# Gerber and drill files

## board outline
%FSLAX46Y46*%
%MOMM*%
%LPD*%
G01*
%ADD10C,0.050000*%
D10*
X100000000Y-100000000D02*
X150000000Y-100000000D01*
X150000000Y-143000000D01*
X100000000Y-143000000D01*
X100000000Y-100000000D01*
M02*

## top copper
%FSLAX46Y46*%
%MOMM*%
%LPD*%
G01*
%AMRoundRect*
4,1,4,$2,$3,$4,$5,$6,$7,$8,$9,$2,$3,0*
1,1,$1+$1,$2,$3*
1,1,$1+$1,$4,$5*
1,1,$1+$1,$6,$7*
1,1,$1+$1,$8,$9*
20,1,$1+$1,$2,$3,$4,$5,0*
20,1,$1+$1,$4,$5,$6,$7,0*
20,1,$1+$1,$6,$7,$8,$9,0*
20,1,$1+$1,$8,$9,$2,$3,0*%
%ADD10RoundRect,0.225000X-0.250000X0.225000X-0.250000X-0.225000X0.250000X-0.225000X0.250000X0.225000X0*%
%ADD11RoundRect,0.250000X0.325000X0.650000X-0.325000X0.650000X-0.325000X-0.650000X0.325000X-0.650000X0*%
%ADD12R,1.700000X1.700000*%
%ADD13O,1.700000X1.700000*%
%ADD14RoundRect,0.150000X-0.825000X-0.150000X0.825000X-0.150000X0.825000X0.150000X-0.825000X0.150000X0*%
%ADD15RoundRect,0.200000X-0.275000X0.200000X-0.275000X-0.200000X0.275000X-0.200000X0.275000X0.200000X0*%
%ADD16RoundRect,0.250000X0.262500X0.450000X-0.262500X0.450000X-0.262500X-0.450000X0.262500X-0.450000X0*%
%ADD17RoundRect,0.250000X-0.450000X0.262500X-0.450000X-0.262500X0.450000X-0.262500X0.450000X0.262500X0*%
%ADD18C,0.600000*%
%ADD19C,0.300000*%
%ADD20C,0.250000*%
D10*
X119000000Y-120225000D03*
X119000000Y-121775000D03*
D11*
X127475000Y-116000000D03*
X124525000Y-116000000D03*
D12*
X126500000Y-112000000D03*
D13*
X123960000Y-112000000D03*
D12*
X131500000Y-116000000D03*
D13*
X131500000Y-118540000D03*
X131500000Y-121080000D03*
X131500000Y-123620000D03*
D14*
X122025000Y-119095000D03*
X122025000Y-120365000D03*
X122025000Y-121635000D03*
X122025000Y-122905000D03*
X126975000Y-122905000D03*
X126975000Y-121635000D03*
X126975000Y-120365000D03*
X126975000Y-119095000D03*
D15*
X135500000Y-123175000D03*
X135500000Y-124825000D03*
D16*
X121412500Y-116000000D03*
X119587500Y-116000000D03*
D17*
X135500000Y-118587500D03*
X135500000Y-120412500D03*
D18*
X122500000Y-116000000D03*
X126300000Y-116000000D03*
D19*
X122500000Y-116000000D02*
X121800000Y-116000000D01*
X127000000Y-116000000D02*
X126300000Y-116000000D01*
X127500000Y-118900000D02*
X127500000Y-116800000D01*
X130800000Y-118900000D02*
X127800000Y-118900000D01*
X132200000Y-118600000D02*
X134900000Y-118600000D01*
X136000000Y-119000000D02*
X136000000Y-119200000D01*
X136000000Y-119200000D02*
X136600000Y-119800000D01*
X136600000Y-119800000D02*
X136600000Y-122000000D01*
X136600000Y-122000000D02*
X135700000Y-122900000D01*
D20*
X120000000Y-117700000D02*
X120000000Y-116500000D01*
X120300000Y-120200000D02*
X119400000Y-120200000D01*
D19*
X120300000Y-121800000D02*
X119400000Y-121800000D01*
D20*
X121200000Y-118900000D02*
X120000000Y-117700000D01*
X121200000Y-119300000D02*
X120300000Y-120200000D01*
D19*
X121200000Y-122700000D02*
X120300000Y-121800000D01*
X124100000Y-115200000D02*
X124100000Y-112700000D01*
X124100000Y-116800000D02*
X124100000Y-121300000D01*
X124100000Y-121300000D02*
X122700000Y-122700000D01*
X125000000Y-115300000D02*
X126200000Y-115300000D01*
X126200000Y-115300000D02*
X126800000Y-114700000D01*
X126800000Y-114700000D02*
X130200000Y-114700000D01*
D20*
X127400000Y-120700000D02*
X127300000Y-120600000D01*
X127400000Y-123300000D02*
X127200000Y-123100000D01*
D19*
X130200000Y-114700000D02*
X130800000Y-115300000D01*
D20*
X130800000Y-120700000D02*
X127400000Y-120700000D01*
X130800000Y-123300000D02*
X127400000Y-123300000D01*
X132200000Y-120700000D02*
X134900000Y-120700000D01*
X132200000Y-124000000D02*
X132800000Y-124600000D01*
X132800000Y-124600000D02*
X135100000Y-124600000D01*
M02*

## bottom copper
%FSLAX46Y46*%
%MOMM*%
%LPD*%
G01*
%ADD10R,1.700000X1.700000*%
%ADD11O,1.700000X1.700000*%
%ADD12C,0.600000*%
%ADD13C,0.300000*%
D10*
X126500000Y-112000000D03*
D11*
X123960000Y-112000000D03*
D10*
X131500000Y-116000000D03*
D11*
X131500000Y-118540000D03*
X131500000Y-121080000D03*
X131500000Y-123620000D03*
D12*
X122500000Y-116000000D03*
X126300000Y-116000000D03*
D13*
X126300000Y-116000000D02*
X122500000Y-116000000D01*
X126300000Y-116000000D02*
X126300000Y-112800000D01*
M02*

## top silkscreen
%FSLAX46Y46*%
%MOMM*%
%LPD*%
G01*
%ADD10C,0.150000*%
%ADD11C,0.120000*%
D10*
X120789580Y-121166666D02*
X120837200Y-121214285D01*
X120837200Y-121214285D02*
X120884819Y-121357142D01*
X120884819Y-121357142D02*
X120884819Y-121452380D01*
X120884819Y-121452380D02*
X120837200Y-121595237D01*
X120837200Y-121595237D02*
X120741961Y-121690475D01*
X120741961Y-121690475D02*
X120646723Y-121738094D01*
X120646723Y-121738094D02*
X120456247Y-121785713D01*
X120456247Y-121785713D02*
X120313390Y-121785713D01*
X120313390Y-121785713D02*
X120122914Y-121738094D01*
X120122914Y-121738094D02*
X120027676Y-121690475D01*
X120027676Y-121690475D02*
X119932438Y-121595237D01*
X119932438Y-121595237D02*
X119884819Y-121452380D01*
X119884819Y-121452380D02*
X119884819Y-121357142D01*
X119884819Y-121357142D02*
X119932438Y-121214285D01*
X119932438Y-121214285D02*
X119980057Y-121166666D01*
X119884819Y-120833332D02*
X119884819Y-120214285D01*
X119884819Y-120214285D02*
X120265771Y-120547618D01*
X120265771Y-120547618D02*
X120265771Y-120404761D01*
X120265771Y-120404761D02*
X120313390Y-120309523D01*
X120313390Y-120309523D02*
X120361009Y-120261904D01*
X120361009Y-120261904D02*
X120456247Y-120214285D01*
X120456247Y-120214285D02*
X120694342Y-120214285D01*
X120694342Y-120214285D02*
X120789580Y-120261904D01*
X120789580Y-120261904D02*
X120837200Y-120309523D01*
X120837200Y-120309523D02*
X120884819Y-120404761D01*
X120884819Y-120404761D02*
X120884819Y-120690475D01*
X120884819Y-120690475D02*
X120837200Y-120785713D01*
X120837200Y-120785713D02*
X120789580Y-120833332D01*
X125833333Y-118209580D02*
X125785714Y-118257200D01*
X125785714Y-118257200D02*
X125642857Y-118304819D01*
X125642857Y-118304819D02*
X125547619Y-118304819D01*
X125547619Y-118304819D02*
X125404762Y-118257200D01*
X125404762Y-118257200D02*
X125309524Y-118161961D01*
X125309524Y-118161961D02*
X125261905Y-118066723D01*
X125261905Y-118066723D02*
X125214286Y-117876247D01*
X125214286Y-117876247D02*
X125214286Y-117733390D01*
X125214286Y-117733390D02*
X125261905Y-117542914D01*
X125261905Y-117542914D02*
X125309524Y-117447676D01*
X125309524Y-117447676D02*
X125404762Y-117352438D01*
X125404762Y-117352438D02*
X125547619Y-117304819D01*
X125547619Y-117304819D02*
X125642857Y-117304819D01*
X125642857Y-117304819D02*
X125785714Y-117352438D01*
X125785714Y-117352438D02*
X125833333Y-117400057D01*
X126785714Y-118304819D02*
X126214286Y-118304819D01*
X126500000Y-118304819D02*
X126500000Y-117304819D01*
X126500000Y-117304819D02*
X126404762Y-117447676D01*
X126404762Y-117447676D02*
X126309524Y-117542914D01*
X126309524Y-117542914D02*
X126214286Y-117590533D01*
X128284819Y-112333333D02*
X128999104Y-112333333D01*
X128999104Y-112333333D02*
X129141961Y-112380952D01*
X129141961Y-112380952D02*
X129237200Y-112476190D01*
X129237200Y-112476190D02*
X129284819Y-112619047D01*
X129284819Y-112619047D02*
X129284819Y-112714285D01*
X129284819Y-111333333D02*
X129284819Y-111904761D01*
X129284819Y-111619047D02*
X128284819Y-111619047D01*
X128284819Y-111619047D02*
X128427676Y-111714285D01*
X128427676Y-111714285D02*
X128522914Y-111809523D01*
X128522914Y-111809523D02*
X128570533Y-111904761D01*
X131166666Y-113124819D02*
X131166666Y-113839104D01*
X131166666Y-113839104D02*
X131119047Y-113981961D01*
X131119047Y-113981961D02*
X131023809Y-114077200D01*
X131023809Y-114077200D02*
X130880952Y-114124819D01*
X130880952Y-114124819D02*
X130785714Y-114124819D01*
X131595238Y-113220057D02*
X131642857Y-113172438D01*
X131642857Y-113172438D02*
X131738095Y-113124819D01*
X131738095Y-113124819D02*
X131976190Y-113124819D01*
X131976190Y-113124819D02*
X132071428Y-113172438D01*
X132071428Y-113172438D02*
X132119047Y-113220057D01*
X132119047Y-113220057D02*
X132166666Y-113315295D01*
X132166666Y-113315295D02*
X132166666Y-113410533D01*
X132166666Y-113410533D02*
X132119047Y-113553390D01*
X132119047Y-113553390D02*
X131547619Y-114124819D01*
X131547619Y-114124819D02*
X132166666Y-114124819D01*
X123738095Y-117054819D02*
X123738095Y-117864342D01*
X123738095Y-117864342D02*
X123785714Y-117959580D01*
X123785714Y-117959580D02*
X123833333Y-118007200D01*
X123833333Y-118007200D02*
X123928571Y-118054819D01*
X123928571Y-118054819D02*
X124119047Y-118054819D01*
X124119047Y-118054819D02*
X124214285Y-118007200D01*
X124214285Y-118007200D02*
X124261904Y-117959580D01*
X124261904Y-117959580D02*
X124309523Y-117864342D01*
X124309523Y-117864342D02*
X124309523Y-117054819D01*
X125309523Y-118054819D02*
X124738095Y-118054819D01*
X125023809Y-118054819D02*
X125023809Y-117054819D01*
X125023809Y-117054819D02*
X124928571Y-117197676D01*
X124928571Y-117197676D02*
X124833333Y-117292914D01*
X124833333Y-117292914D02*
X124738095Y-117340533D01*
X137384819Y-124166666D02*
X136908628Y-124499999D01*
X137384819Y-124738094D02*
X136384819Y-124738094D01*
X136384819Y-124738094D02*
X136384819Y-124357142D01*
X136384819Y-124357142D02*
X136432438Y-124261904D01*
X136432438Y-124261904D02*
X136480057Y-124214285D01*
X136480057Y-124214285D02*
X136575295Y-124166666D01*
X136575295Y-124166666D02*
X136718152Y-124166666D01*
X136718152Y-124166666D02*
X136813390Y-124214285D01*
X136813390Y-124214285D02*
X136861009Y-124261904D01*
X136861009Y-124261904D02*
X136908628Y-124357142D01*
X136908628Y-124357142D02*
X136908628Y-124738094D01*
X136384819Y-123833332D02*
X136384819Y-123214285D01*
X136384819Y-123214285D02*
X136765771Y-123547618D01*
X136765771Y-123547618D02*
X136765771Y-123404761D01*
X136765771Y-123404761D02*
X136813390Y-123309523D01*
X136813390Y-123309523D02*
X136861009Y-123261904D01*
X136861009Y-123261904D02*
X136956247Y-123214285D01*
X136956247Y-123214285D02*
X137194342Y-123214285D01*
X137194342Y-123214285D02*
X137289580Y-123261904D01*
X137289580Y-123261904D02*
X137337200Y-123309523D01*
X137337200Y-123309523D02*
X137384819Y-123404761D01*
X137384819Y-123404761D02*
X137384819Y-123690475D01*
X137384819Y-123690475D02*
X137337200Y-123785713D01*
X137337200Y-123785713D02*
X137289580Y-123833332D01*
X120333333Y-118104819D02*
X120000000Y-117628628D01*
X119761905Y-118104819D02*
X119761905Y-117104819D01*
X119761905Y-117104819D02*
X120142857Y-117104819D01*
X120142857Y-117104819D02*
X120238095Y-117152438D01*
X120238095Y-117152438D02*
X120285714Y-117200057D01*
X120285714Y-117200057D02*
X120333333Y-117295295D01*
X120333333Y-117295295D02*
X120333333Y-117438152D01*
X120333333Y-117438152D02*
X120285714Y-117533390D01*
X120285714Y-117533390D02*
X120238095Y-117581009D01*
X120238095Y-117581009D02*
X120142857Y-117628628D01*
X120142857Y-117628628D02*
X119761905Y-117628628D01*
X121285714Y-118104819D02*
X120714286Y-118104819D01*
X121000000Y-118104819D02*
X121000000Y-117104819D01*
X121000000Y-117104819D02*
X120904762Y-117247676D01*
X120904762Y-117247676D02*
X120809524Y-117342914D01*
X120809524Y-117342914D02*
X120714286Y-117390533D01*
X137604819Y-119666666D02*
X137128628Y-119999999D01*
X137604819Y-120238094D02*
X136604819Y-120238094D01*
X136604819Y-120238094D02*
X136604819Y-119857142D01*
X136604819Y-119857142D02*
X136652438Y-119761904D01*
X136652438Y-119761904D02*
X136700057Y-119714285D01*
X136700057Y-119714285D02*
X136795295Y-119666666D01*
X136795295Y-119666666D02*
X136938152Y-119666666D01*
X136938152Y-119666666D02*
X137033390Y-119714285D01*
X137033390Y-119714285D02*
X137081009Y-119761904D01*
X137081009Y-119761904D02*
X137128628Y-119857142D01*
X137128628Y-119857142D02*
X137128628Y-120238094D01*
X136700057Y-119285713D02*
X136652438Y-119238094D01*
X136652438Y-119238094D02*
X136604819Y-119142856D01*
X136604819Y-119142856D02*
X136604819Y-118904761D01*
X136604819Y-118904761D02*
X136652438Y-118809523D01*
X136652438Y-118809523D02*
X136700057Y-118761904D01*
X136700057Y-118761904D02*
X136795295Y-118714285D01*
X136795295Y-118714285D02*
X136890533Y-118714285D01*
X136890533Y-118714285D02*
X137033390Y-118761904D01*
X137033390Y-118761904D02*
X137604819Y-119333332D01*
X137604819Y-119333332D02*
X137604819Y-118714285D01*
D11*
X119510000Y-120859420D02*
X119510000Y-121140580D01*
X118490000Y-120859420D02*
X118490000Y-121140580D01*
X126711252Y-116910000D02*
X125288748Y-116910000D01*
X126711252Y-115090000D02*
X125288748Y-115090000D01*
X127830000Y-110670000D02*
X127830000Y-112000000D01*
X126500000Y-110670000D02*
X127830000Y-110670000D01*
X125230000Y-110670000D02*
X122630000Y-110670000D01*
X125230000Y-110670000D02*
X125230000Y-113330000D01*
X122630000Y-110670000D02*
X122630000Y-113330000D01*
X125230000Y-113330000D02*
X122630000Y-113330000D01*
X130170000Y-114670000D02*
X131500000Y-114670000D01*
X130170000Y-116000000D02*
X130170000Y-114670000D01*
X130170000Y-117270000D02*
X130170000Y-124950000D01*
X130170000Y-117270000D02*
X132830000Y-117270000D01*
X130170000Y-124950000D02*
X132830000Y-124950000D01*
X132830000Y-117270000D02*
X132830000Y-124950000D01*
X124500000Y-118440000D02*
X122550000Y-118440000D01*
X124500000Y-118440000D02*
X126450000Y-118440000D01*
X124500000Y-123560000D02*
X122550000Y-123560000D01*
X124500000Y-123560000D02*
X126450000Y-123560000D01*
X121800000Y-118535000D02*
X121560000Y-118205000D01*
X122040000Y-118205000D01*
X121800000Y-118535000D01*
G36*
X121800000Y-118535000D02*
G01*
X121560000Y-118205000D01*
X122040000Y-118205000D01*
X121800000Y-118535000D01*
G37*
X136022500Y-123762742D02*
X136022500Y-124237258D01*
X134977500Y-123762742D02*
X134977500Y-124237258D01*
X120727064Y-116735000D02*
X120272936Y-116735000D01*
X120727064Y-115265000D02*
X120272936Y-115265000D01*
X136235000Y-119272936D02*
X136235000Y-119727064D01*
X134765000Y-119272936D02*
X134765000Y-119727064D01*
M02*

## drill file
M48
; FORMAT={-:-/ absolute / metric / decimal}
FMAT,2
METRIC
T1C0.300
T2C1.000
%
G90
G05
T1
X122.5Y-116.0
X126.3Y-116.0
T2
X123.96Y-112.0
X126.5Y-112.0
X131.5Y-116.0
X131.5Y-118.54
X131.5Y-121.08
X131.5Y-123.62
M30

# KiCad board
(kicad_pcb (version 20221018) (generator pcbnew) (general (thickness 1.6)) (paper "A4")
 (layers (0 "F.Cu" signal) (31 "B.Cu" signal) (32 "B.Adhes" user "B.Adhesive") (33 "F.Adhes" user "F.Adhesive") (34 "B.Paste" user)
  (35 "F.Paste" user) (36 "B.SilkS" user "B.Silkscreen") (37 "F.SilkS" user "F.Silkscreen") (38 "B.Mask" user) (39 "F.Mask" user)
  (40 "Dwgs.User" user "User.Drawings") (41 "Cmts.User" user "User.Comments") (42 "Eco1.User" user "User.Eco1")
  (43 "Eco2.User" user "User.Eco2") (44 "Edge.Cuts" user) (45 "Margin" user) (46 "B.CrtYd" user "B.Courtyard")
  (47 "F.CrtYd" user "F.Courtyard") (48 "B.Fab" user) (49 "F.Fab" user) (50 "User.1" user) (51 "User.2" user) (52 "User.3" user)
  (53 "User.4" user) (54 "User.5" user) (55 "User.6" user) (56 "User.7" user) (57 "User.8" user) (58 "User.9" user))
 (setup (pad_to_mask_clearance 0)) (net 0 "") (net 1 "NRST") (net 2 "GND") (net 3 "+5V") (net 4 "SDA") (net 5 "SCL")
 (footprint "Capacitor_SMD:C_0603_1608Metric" (layer "F.Cu") (at 119 121 -90)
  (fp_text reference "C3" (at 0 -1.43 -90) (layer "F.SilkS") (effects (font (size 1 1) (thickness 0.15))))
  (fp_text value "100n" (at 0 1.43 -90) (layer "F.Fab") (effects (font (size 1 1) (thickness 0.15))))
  (fp_line (start -0.14058 -0.51) (end 0.14058 -0.51) (stroke (width 0.12) (type solid)) (layer "F.SilkS"))
  (fp_line (start -0.14058 0.51) (end 0.14058 0.51) (stroke (width 0.12) (type solid)) (layer "F.SilkS"))
  (pad "1" smd roundrect (at -0.775 0 270) (size 0.9 0.95) (layers "F.Cu" "F.Paste" "F.Mask") (roundrect_rratio 0.25) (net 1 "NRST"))
  (pad "2" smd roundrect (at 0.775 0 270) (size 0.9 0.95) (layers "F.Cu" "F.Paste" "F.Mask") (roundrect_rratio 0.25) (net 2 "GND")))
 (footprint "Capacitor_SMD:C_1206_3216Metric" (layer "F.Cu") (at 126 116 180)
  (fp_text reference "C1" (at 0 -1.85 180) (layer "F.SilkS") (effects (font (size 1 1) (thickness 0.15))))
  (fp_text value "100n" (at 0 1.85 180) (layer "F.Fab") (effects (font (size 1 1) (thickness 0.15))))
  (fp_line (start -0.711252 -0.91) (end 0.711252 -0.91) (stroke (width 0.12) (type solid)) (layer "F.SilkS"))
  (fp_line (start -0.711252 0.91) (end 0.711252 0.91) (stroke (width 0.12) (type solid)) (layer "F.SilkS"))
  (pad "1" smd roundrect (at -1.475 0 180) (size 1.15 1.8) (layers "F.Cu" "F.Paste" "F.Mask") (roundrect_rratio 0.217391) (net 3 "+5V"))
  (pad "2" smd roundrect (at 1.475 0 180) (size 1.15 1.8) (layers "F.Cu" "F.Paste" "F.Mask") (roundrect_rratio 0.217391) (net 2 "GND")))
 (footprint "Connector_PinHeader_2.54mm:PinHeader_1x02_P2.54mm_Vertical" (layer "F.Cu") (at 126.5 112 -90)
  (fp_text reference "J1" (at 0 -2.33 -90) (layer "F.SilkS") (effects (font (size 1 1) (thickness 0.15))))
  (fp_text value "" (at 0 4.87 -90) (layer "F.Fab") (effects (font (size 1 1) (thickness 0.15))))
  (fp_line (start -1.33 -1.33) (end 0 -1.33) (stroke (width 0.12) (type solid)) (layer "F.SilkS"))
  (fp_line (start -1.33 0) (end -1.33 -1.33) (stroke (width 0.12) (type solid)) (layer "F.SilkS"))
  (fp_line (start -1.33 1.27) (end -1.33 3.87) (stroke (width 0.12) (type solid)) (layer "F.SilkS"))
  (fp_line (start -1.33 1.27) (end 1.33 1.27) (stroke (width 0.12) (type solid)) (layer "F.SilkS"))
  (fp_line (start -1.33 3.87) (end 1.33 3.87) (stroke (width 0.12) (type solid)) (layer "F.SilkS"))
  (fp_line (start 1.33 1.27) (end 1.33 3.87) (stroke (width 0.12) (type solid)) (layer "F.SilkS"))
  (pad "1" thru_hole rect (at 0 0 270) (size 1.7 1.7) (drill 1) (layers "*.Cu" "*.Mask") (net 3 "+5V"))
  (pad "2" thru_hole oval (at 0 2.54 270) (size 1.7 1.7) (drill 1) (layers "*.Cu" "*.Mask") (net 2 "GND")))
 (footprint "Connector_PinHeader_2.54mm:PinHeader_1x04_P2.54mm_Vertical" (layer "F.Cu") (at 131.5 116)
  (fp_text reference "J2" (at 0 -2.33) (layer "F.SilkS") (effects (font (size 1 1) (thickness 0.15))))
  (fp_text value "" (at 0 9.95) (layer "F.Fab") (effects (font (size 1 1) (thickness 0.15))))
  (fp_line (start -1.33 -1.33) (end 0 -1.33) (stroke (width 0.12) (type solid)) (layer "F.SilkS"))
  (fp_line (start -1.33 0) (end -1.33 -1.33) (stroke (width 0.12) (type solid)) (layer "F.SilkS"))
  (fp_line (start -1.33 1.27) (end -1.33 8.95) (stroke (width 0.12) (type solid)) (layer "F.SilkS"))
  (fp_line (start -1.33 1.27) (end 1.33 1.27) (stroke (width 0.12) (type solid)) (layer "F.SilkS"))
  (fp_line (start -1.33 8.95) (end 1.33 8.95) (stroke (width 0.12) (type solid)) (layer "F.SilkS"))
  (fp_line (start 1.33 1.27) (end 1.33 8.95) (stroke (width 0.12) (type solid)) (layer "F.SilkS"))
  (pad "1" thru_hole rect (at 0 0) (size 1.7 1.7) (drill 1) (layers "*.Cu" "*.Mask") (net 2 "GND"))
  (pad "2" thru_hole oval (at 0 2.54) (size 1.7 1.7) (drill 1) (layers "*.Cu" "*.Mask") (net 3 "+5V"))
  (pad "3" thru_hole oval (at 0 5.08) (size 1.7 1.7) (drill 1) (layers "*.Cu" "*.Mask") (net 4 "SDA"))
  (pad "4" thru_hole oval (at 0 7.62) (size 1.7 1.7) (drill 1) (layers "*.Cu" "*.Mask") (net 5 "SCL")))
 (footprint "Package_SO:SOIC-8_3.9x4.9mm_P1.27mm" (layer "F.Cu") (at 124.5 121)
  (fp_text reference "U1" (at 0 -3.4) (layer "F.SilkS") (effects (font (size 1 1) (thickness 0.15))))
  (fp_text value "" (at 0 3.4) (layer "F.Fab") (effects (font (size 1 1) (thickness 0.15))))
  (fp_line (start 0 -2.56) (end -1.95 -2.56) (stroke (width 0.12) (type solid)) (layer "F.SilkS"))
  (fp_line (start 0 -2.56) (end 1.95 -2.56) (stroke (width 0.12) (type solid)) (layer "F.SilkS"))
  (fp_line (start 0 2.56) (end -1.95 2.56) (stroke (width 0.12) (type solid)) (layer "F.SilkS"))
  (fp_line (start 0 2.56) (end 1.95 2.56) (stroke (width 0.12) (type solid)) (layer "F.SilkS"))
  (fp_poly
   (pts (xy -2.7 -2.465) (xy -2.94 -2.795) (xy -2.46 -2.795) (xy -2.7 -2.465)) (stroke (width 0.12) (type solid)) (fill solid)
   (layer "F.SilkS"))
  (pad "1" smd roundrect (at -2.475 -1.905) (size 1.95 0.6) (layers "F.Cu" "F.Paste" "F.Mask") (roundrect_rratio 0.25) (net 1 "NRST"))
  (pad "2" smd roundrect (at -2.475 -0.635) (size 1.95 0.6) (layers "F.Cu" "F.Paste" "F.Mask") (roundrect_rratio 0.25))
  (pad "3" smd roundrect (at -2.475 0.635) (size 1.95 0.6) (layers "F.Cu" "F.Paste" "F.Mask") (roundrect_rratio 0.25))
  (pad "4" smd roundrect (at -2.475 1.905) (size 1.95 0.6) (layers "F.Cu" "F.Paste" "F.Mask") (roundrect_rratio 0.25) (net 2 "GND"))
  (pad "5" smd roundrect (at 2.475 1.905) (size 1.95 0.6) (layers "F.Cu" "F.Paste" "F.Mask") (roundrect_rratio 0.25) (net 5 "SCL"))
  (pad "6" smd roundrect (at 2.475 0.635) (size 1.95 0.6) (layers "F.Cu" "F.Paste" "F.Mask") (roundrect_rratio 0.25))
  (pad "7" smd roundrect (at 2.475 -0.635) (size 1.95 0.6) (layers "F.Cu" "F.Paste" "F.Mask") (roundrect_rratio 0.25) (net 4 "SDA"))
  (pad "8" smd roundrect (at 2.475 -1.905) (size 1.95 0.6) (layers "F.Cu" "F.Paste" "F.Mask") (roundrect_rratio 0.25) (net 3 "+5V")))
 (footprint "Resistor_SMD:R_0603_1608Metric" (layer "F.Cu") (at 135.5 124 -90)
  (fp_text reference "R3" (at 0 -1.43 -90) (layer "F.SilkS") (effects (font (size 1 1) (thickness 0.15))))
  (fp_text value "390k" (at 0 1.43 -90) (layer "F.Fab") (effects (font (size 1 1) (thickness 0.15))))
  (fp_line (start -0.237258 -0.5225) (end 0.237258 -0.5225) (stroke (width 0.12) (type solid)) (layer "F.SilkS"))
  (fp_line (start -0.237258 0.5225) (end 0.237258 0.5225) (stroke (width 0.12) (type solid)) (layer "F.SilkS"))
  (pad "1" smd roundrect (at -0.825 0 270) (size 0.8 0.95) (layers "F.Cu" "F.Paste" "F.Mask") (roundrect_rratio 0.25) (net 3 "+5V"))
  (pad "2" smd roundrect (at 0.825 0 270) (size 0.8 0.95) (layers "F.Cu" "F.Paste" "F.Mask") (roundrect_rratio 0.25) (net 5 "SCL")))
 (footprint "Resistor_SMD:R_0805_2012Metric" (layer "F.Cu") (at 120.5 116 180)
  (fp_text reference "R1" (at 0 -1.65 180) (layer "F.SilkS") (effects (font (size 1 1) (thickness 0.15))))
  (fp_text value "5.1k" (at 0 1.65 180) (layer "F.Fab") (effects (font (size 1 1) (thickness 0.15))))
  (fp_line (start -0.227064 -0.735) (end 0.227064 -0.735) (stroke (width 0.12) (type solid)) (layer "F.SilkS"))
  (fp_line (start -0.227064 0.735) (end 0.227064 0.735) (stroke (width 0.12) (type solid)) (layer "F.SilkS"))
  (pad "1" smd roundrect (at -0.9125 0 180) (size 1.025 1.4) (layers "F.Cu" "F.Paste" "F.Mask") (roundrect_rratio 0.243902) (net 3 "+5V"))
  (pad "2" smd roundrect (at 0.9125 0 180) (size 1.025 1.4) (layers "F.Cu" "F.Paste" "F.Mask") (roundrect_rratio 0.243902) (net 1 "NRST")))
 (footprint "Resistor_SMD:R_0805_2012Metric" (layer "F.Cu") (at 135.5 119.5 -90)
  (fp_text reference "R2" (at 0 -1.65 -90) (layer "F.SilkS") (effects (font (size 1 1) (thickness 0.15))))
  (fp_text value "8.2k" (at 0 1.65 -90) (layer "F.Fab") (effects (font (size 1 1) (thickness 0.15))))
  (fp_line (start -0.227064 -0.735) (end 0.227064 -0.735) (stroke (width 0.12) (type solid)) (layer "F.SilkS"))
  (fp_line (start -0.227064 0.735) (end 0.227064 0.735) (stroke (width 0.12) (type solid)) (layer "F.SilkS"))
  (pad "1" smd roundrect (at -0.9125 0 270) (size 1.025 1.4) (layers "F.Cu" "F.Paste" "F.Mask") (roundrect_rratio 0.243902) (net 3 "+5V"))
  (pad "2" smd roundrect (at 0.9125 0 270) (size 1.025 1.4) (layers "F.Cu" "F.Paste" "F.Mask") (roundrect_rratio 0.243902) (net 4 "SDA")))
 (gr_rect (start 100 100) (end 150 143) (stroke (width 0.05) (type default)) (fill none) (layer "Edge.Cuts"))
 (segment (start 122.5 116) (end 121.8 116) (width 0.3) (layer "F.Cu") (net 3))
 (segment (start 127 116) (end 126.3 116) (width 0.3) (layer "F.Cu") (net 3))
 (segment (start 127.5 118.9) (end 127.5 116.8) (width 0.3) (layer "F.Cu") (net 3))
 (segment (start 130.8 118.9) (end 127.8 118.9) (width 0.3) (layer "F.Cu") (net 3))
 (segment (start 132.2 118.6) (end 134.9 118.6) (width 0.3) (layer "F.Cu") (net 3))
 (segment (start 136 119) (end 136 119.2) (width 0.3) (layer "F.Cu") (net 3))
 (segment (start 136 119.2) (end 136.6 119.8) (width 0.3) (layer "F.Cu") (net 3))
 (segment (start 136.6 119.8) (end 136.6 122) (width 0.3) (layer "F.Cu") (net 3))
 (segment (start 136.6 122) (end 135.7 122.9) (width 0.3) (layer "F.Cu") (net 3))
 (via (at 122.5 116) (size 0.6) (drill 0.3) (layers "F.Cu" "B.Cu") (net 3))
 (via (at 126.3 116) (size 0.6) (drill 0.3) (layers "F.Cu" "B.Cu") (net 3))
 (segment (start 120 117.7) (end 120 116.5) (width 0.25) (layer "F.Cu") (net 1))
 (segment (start 120.3 120.2) (end 119.4 120.2) (width 0.25) (layer "F.Cu") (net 1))
 (segment (start 120.3 121.8) (end 119.4 121.8) (width 0.3) (layer "F.Cu") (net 2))
 (segment (start 121.2 118.9) (end 120 117.7) (width 0.25) (layer "F.Cu") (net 1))
 (segment (start 121.2 119.3) (end 120.3 120.2) (width 0.25) (layer "F.Cu") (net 1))
 (segment (start 121.2 122.7) (end 120.3 121.8) (width 0.3) (layer "F.Cu") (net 2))
 (segment (start 124.1 115.2) (end 124.1 112.7) (width 0.3) (layer "F.Cu") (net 2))
 (segment (start 124.1 116.8) (end 124.1 121.3) (width 0.3) (layer "F.Cu") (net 2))
 (segment (start 124.1 121.3) (end 122.7 122.7) (width 0.3) (layer "F.Cu") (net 2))
 (segment (start 125 115.3) (end 126.2 115.3) (width 0.3) (layer "F.Cu") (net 2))
 (segment (start 126.2 115.3) (end 126.8 114.7) (width 0.3) (layer "F.Cu") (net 2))
 (segment (start 126.3 116) (end 122.5 116) (width 0.3) (layer "B.Cu") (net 3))
 (segment (start 126.3 116) (end 126.3 112.8) (width 0.3) (layer "B.Cu") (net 3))
 (segment (start 126.8 114.7) (end 130.2 114.7) (width 0.3) (layer "F.Cu") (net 2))
 (segment (start 127.4 120.7) (end 127.3 120.6) (width 0.25) (layer "F.Cu") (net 4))
 (segment (start 127.4 123.3) (end 127.2 123.1) (width 0.25) (layer "F.Cu") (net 5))
 (segment (start 130.2 114.7) (end 130.8 115.3) (width 0.3) (layer "F.Cu") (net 2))
 (segment (start 130.8 120.7) (end 127.4 120.7) (width 0.25) (layer "F.Cu") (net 4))
 (segment (start 130.8 123.3) (end 127.4 123.3) (width 0.25) (layer "F.Cu") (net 5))
 (segment (start 132.2 120.7) (end 134.9 120.7) (width 0.25) (layer "F.Cu") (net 4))
 (segment (start 132.2 124) (end 132.8 124.6) (width 0.25) (layer "F.Cu") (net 5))
 (segment (start 132.8 124.6) (end 135.1 124.6) (width 0.25) (layer "F.Cu") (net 5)))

